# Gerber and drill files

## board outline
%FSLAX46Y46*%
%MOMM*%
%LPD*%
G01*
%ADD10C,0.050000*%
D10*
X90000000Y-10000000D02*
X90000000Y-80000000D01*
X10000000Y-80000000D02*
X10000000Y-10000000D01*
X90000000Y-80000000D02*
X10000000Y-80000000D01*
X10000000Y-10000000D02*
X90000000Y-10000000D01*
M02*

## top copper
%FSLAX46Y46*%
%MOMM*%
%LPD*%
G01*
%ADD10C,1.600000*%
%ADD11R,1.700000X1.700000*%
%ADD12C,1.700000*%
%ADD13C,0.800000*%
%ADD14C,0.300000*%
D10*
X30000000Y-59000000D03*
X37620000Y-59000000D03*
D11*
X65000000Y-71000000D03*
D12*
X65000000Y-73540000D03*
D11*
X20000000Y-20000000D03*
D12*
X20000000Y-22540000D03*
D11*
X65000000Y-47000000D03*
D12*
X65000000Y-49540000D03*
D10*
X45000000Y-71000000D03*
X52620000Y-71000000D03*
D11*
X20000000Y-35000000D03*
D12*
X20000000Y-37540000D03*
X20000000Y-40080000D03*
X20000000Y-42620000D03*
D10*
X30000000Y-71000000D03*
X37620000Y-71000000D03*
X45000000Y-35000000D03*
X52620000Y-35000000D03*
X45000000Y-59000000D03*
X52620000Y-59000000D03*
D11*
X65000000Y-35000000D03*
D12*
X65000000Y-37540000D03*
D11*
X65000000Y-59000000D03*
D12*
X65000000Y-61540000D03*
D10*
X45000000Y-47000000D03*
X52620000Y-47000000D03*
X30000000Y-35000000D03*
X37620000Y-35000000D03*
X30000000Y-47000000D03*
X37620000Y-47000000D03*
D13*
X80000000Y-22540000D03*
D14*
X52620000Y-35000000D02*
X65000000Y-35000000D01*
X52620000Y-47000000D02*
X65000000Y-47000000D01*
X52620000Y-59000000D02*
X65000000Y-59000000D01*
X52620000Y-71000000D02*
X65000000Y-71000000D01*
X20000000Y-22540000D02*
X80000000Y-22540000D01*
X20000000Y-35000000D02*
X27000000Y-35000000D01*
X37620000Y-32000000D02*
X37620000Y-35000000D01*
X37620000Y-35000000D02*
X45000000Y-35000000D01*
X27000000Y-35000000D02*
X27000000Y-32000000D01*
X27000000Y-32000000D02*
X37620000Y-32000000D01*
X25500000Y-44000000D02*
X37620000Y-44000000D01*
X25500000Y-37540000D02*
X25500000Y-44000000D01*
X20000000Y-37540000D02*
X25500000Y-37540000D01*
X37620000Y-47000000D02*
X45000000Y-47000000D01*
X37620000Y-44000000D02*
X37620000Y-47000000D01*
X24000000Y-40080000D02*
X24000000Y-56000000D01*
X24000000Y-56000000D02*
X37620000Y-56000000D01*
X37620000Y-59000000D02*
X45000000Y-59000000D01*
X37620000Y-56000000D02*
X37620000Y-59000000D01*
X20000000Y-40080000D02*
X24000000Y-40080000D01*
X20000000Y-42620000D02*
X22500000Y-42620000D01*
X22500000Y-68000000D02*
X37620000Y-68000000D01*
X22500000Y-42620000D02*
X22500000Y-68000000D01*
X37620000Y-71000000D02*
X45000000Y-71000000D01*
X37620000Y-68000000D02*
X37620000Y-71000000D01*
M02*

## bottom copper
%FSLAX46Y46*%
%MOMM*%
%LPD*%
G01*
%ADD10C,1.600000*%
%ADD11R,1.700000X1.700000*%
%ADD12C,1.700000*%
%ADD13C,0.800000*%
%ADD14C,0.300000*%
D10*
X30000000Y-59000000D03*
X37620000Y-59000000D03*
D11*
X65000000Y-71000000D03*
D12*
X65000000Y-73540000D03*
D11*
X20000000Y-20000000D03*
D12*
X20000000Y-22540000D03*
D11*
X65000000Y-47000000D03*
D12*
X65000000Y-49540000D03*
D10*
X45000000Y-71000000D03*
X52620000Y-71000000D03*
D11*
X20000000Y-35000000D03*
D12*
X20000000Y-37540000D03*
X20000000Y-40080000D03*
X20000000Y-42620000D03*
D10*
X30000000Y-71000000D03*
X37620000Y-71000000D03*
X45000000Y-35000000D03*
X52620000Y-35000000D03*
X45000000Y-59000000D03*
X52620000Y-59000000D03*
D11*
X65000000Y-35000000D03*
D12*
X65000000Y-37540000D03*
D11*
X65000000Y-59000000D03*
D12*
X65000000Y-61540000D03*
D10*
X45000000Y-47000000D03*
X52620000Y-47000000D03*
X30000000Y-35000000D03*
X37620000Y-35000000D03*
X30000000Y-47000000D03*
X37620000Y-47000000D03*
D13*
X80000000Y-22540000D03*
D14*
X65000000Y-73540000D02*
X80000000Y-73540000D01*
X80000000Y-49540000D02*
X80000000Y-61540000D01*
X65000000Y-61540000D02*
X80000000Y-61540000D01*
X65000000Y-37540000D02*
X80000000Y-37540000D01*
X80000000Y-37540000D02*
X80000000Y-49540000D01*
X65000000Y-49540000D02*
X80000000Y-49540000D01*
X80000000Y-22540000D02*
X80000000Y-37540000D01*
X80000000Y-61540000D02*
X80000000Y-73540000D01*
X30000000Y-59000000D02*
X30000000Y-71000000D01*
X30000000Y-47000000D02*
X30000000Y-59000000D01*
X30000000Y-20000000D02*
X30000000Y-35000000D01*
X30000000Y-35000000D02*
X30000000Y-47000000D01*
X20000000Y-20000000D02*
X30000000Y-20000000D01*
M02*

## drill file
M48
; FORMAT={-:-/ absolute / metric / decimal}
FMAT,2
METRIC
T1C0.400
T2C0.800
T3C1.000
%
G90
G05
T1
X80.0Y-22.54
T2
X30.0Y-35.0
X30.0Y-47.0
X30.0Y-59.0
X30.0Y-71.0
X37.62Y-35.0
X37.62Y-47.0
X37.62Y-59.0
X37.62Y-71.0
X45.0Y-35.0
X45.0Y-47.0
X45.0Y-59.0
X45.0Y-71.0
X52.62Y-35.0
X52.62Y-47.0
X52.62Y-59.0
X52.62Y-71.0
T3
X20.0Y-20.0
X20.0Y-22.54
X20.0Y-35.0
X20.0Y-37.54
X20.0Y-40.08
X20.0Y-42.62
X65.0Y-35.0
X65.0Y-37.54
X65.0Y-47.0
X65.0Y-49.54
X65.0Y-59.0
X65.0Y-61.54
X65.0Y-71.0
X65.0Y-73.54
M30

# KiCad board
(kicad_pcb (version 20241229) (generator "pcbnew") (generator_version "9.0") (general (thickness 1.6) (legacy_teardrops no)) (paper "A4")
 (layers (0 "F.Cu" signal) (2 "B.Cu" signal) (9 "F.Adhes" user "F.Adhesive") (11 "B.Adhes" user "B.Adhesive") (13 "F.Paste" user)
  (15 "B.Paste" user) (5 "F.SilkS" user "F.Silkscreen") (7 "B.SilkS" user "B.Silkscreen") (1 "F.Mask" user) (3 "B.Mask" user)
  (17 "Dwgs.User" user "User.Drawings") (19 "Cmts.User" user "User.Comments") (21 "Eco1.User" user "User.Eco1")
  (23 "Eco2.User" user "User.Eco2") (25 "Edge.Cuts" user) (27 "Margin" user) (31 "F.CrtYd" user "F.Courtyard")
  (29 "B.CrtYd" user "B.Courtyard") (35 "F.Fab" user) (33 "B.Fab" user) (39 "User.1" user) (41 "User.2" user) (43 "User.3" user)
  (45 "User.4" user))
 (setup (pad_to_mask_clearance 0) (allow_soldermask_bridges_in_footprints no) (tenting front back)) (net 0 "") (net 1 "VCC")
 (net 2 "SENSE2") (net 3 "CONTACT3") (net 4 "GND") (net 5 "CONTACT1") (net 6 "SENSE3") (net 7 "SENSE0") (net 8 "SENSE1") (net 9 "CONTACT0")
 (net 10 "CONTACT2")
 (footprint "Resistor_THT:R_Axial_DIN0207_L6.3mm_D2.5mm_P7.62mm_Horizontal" (layer "F.Cu") (at 30 59)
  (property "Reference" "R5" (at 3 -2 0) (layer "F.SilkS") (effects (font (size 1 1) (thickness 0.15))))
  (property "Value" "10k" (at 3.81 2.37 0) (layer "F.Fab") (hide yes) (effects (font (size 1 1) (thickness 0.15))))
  (pad "1" thru_hole circle (at 0 0) (size 1.6 1.6) (drill 0.8) (layers "*.Cu" "*.Mask") (remove_unused_layers no) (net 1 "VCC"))
  (pad "2" thru_hole circle (at 7.62 0) (size 1.6 1.6) (drill 0.8) (layers "*.Cu" "*.Mask") (remove_unused_layers no) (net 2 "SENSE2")))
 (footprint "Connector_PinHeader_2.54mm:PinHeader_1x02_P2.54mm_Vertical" (layer "F.Cu") (at 65 71)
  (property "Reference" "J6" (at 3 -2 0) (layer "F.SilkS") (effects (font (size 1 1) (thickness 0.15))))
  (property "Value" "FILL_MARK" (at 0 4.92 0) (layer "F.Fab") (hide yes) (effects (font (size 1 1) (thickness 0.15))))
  (pad "1" thru_hole rect (at 0 0) (size 1.7 1.7) (drill 1) (layers "*.Cu" "*.Mask") (remove_unused_layers no) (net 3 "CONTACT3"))
  (pad "2" thru_hole circle (at 0 2.54) (size 1.7 1.7) (drill 1) (layers "*.Cu" "*.Mask") (remove_unused_layers no) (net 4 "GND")))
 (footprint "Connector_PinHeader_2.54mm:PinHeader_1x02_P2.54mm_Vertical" (layer "F.Cu") (at 20 20)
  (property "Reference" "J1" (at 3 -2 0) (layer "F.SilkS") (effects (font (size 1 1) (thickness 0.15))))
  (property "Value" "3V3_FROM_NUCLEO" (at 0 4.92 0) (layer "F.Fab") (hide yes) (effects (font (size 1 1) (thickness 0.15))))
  (pad "1" thru_hole rect (at 0 0) (size 1.7 1.7) (drill 1) (layers "*.Cu" "*.Mask") (remove_unused_layers no) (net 1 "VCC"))
  (pad "2" thru_hole circle (at 0 2.54) (size 1.7 1.7) (drill 1) (layers "*.Cu" "*.Mask") (remove_unused_layers no) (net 4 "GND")))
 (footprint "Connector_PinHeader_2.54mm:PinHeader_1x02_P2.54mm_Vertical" (layer "F.Cu") (at 65 47)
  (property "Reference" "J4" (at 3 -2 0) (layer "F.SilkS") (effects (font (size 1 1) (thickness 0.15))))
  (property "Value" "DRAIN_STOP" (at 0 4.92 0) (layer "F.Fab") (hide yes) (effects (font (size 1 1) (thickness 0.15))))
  (pad "1" thru_hole rect (at 0 0) (size 1.7 1.7) (drill 1) (layers "*.Cu" "*.Mask") (remove_unused_layers no) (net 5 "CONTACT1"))
  (pad "2" thru_hole circle (at 0 2.54) (size 1.7 1.7) (drill 1) (layers "*.Cu" "*.Mask") (remove_unused_layers no) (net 4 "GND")))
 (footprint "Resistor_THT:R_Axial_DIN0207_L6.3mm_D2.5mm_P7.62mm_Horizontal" (layer "F.Cu") (at 45 71)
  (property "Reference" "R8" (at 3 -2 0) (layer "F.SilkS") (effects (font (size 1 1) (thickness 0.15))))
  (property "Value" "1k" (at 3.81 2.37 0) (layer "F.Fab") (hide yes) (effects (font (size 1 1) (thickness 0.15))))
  (pad "1" thru_hole circle (at 0 0) (size 1.6 1.6) (drill 0.8) (layers "*.Cu" "*.Mask") (remove_unused_layers no) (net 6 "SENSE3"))
  (pad "2" thru_hole circle (at 7.62 0) (size 1.6 1.6) (drill 0.8) (layers "*.Cu" "*.Mask") (remove_unused_layers no) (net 3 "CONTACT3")))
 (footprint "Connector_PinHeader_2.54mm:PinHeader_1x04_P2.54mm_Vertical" (layer "F.Cu") (at 20 35)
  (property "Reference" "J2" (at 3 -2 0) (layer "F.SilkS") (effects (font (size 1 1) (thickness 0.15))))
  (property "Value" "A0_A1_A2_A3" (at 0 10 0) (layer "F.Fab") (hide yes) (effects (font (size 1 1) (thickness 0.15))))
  (pad "1" thru_hole rect (at 0 0) (size 1.7 1.7) (drill 1) (layers "*.Cu" "*.Mask") (remove_unused_layers no) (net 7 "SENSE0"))
  (pad "2" thru_hole circle (at 0 2.54) (size 1.7 1.7) (drill 1) (layers "*.Cu" "*.Mask") (remove_unused_layers no) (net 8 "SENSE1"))
  (pad "3" thru_hole circle (at 0 5.08) (size 1.7 1.7) (drill 1) (layers "*.Cu" "*.Mask") (remove_unused_layers no) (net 2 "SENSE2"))
  (pad "4" thru_hole circle (at 0 7.62) (size 1.7 1.7) (drill 1) (layers "*.Cu" "*.Mask") (remove_unused_layers no) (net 6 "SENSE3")))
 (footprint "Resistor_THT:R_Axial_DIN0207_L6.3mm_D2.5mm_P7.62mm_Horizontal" (layer "F.Cu") (at 30 71)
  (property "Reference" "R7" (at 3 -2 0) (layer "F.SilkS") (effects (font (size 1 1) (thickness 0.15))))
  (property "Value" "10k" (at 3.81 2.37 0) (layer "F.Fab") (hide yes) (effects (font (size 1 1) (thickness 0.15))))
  (pad "1" thru_hole circle (at 0 0) (size 1.6 1.6) (drill 0.8) (layers "*.Cu" "*.Mask") (remove_unused_layers no) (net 1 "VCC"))
  (pad "2" thru_hole circle (at 7.62 0) (size 1.6 1.6) (drill 0.8) (layers "*.Cu" "*.Mask") (remove_unused_layers no) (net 6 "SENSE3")))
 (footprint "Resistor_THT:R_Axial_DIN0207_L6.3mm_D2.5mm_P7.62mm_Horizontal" (layer "F.Cu") (at 45 35)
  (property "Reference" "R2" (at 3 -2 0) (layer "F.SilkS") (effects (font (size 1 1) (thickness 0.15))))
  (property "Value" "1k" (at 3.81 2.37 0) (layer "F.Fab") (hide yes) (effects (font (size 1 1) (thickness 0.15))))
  (pad "1" thru_hole circle (at 0 0) (size 1.6 1.6) (drill 0.8) (layers "*.Cu" "*.Mask") (remove_unused_layers no) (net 7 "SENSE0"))
  (pad "2" thru_hole circle (at 7.62 0) (size 1.6 1.6) (drill 0.8) (layers "*.Cu" "*.Mask") (remove_unused_layers no) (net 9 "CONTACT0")))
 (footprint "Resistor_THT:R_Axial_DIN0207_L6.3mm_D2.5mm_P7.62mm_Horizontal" (layer "F.Cu") (at 45 59)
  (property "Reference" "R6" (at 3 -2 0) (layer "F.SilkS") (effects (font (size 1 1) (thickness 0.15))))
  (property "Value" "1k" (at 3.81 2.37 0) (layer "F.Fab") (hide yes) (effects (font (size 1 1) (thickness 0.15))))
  (pad "1" thru_hole circle (at 0 0) (size 1.6 1.6) (drill 0.8) (layers "*.Cu" "*.Mask") (remove_unused_layers no) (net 2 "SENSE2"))
  (pad "2" thru_hole circle (at 7.62 0) (size 1.6 1.6) (drill 0.8) (layers "*.Cu" "*.Mask") (remove_unused_layers no) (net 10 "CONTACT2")))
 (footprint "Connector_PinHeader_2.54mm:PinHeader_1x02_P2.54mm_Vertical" (layer "F.Cu") (at 65 35)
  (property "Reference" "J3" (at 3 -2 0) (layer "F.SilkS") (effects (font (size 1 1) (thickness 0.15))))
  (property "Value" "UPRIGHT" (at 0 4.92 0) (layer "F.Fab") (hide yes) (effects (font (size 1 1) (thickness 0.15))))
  (pad "1" thru_hole rect (at 0 0) (size 1.7 1.7) (drill 1) (layers "*.Cu" "*.Mask") (remove_unused_layers no) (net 9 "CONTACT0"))
  (pad "2" thru_hole circle (at 0 2.54) (size 1.7 1.7) (drill 1) (layers "*.Cu" "*.Mask") (remove_unused_layers no) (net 4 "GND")))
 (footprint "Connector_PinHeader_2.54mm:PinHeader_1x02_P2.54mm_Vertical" (layer "F.Cu") (at 65 59)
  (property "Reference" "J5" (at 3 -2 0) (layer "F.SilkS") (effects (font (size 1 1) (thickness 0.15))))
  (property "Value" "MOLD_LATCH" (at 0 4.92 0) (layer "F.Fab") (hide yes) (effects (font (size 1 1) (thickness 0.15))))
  (pad "1" thru_hole rect (at 0 0) (size 1.7 1.7) (drill 1) (layers "*.Cu" "*.Mask") (remove_unused_layers no) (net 10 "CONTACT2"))
  (pad "2" thru_hole circle (at 0 2.54) (size 1.7 1.7) (drill 1) (layers "*.Cu" "*.Mask") (remove_unused_layers no) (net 4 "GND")))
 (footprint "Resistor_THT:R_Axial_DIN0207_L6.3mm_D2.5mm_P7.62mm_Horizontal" (layer "F.Cu") (at 45 47)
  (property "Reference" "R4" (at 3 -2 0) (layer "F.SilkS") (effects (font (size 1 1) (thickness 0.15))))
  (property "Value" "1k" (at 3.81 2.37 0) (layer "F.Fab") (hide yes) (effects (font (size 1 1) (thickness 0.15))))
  (pad "1" thru_hole circle (at 0 0) (size 1.6 1.6) (drill 0.8) (layers "*.Cu" "*.Mask") (remove_unused_layers no) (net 8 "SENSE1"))
  (pad "2" thru_hole circle (at 7.62 0) (size 1.6 1.6) (drill 0.8) (layers "*.Cu" "*.Mask") (remove_unused_layers no) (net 5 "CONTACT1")))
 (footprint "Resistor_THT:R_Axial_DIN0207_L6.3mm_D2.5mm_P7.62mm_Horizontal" (layer "F.Cu") (at 30 35)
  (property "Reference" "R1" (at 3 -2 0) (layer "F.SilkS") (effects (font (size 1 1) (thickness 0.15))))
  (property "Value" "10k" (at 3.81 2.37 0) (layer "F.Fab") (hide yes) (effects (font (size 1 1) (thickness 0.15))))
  (pad "1" thru_hole circle (at 0 0) (size 1.6 1.6) (drill 0.8) (layers "*.Cu" "*.Mask") (remove_unused_layers no) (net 1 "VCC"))
  (pad "2" thru_hole circle (at 7.62 0) (size 1.6 1.6) (drill 0.8) (layers "*.Cu" "*.Mask") (remove_unused_layers no) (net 7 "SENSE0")))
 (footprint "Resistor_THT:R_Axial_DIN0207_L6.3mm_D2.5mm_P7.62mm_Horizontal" (layer "F.Cu") (at 30 47)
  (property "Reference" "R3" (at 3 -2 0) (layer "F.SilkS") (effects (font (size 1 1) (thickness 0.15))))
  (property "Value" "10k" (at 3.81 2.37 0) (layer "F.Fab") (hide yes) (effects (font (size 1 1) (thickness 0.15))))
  (pad "1" thru_hole circle (at 0 0) (size 1.6 1.6) (drill 0.8) (layers "*.Cu" "*.Mask") (remove_unused_layers no) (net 1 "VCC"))
  (pad "2" thru_hole circle (at 7.62 0) (size 1.6 1.6) (drill 0.8) (layers "*.Cu" "*.Mask") (remove_unused_layers no) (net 8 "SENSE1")))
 (gr_line (start 90 10) (end 90 80) (stroke (width 0.05) (type default)) (layer "Edge.Cuts"))
 (gr_line (start 10 80) (end 10 10) (stroke (width 0.05) (type default)) (layer "Edge.Cuts"))
 (gr_line (start 90 80) (end 10 80) (stroke (width 0.05) (type default)) (layer "Edge.Cuts"))
 (gr_line (start 10 10) (end 90 10) (stroke (width 0.05) (type default)) (layer "Edge.Cuts"))
 (segment (start 52.62 35) (end 65 35) (width 0.3) (layer "F.Cu") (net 9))
 (segment (start 52.62 47) (end 65 47) (width 0.3) (layer "F.Cu") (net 5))
 (segment (start 52.62 59) (end 65 59) (width 0.3) (layer "F.Cu") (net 10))
 (segment (start 52.62 71) (end 65 71) (width 0.3) (layer "F.Cu") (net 3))
 (segment (start 20 22.54) (end 80 22.54) (width 0.3) (layer "F.Cu") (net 4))
 (via (at 80 22.54) (size 0.8) (drill 0.4) (layers "F.Cu" "B.Cu") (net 4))
 (segment (start 65 73.54) (end 80 73.54) (width 0.3) (layer "B.Cu") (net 4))
 (segment (start 80 49.54) (end 80 61.54) (width 0.3) (layer "B.Cu") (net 4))
 (segment (start 65 61.54) (end 80 61.54) (width 0.3) (layer "B.Cu") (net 4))
 (segment (start 65 37.54) (end 80 37.54) (width 0.3) (layer "B.Cu") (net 4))
 (segment (start 80 37.54) (end 80 49.54) (width 0.3) (layer "B.Cu") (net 4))
 (segment (start 65 49.54) (end 80 49.54) (width 0.3) (layer "B.Cu") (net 4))
 (segment (start 80 22.54) (end 80 37.54) (width 0.3) (layer "B.Cu") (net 4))
 (segment (start 80 61.54) (end 80 73.54) (width 0.3) (layer "B.Cu") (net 4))
 (segment (start 20 35) (end 27 35) (width 0.3) (layer "F.Cu") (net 7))
 (segment (start 37.62 32) (end 37.62 35) (width 0.3) (layer "F.Cu") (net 7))
 (segment (start 37.62 35) (end 45 35) (width 0.3) (layer "F.Cu") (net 7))
 (segment (start 27 35) (end 27 32) (width 0.3) (layer "F.Cu") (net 7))
 (segment (start 27 32) (end 37.62 32) (width 0.3) (layer "F.Cu") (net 7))
 (segment (start 25.5 44) (end 37.62 44) (width 0.3) (layer "F.Cu") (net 8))
 (segment (start 25.5 37.54) (end 25.5 44) (width 0.3) (layer "F.Cu") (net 8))
 (segment (start 20 37.54) (end 25.5 37.54) (width 0.3) (layer "F.Cu") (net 8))
 (segment (start 37.62 47) (end 45 47) (width 0.3) (layer "F.Cu") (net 8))
 (segment (start 37.62 44) (end 37.62 47) (width 0.3) (layer "F.Cu") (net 8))
 (segment (start 24 40.08) (end 24 56) (width 0.3) (layer "F.Cu") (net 2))
 (segment (start 24 56) (end 37.62 56) (width 0.3) (layer "F.Cu") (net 2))
 (segment (start 37.62 59) (end 45 59) (width 0.3) (layer "F.Cu") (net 2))
 (segment (start 37.62 56) (end 37.62 59) (width 0.3) (layer "F.Cu") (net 2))
 (segment (start 20 40.08) (end 24 40.08) (width 0.3) (layer "F.Cu") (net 2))
 (segment (start 20 42.62) (end 22.5 42.62) (width 0.3) (layer "F.Cu") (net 6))
 (segment (start 22.5 68) (end 37.62 68) (width 0.3) (layer "F.Cu") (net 6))
 (segment (start 22.5 42.62) (end 22.5 68) (width 0.3) (layer "F.Cu") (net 6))
 (segment (start 37.62 71) (end 45 71) (width 0.3) (layer "F.Cu") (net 6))
 (segment (start 37.62 68) (end 37.62 71) (width 0.3) (layer "F.Cu") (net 6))
 (segment (start 30 59) (end 30 71) (width 0.3) (layer "B.Cu") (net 1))
 (segment (start 30 47) (end 30 59) (width 0.3) (layer "B.Cu") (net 1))
 (segment (start 30 20) (end 30 35) (width 0.3) (layer "B.Cu") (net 1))
 (segment (start 30 35) (end 30 47) (width 0.3) (layer "B.Cu") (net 1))
 (segment (start 20 20) (end 30 20) (width 0.3) (layer "B.Cu") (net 1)))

